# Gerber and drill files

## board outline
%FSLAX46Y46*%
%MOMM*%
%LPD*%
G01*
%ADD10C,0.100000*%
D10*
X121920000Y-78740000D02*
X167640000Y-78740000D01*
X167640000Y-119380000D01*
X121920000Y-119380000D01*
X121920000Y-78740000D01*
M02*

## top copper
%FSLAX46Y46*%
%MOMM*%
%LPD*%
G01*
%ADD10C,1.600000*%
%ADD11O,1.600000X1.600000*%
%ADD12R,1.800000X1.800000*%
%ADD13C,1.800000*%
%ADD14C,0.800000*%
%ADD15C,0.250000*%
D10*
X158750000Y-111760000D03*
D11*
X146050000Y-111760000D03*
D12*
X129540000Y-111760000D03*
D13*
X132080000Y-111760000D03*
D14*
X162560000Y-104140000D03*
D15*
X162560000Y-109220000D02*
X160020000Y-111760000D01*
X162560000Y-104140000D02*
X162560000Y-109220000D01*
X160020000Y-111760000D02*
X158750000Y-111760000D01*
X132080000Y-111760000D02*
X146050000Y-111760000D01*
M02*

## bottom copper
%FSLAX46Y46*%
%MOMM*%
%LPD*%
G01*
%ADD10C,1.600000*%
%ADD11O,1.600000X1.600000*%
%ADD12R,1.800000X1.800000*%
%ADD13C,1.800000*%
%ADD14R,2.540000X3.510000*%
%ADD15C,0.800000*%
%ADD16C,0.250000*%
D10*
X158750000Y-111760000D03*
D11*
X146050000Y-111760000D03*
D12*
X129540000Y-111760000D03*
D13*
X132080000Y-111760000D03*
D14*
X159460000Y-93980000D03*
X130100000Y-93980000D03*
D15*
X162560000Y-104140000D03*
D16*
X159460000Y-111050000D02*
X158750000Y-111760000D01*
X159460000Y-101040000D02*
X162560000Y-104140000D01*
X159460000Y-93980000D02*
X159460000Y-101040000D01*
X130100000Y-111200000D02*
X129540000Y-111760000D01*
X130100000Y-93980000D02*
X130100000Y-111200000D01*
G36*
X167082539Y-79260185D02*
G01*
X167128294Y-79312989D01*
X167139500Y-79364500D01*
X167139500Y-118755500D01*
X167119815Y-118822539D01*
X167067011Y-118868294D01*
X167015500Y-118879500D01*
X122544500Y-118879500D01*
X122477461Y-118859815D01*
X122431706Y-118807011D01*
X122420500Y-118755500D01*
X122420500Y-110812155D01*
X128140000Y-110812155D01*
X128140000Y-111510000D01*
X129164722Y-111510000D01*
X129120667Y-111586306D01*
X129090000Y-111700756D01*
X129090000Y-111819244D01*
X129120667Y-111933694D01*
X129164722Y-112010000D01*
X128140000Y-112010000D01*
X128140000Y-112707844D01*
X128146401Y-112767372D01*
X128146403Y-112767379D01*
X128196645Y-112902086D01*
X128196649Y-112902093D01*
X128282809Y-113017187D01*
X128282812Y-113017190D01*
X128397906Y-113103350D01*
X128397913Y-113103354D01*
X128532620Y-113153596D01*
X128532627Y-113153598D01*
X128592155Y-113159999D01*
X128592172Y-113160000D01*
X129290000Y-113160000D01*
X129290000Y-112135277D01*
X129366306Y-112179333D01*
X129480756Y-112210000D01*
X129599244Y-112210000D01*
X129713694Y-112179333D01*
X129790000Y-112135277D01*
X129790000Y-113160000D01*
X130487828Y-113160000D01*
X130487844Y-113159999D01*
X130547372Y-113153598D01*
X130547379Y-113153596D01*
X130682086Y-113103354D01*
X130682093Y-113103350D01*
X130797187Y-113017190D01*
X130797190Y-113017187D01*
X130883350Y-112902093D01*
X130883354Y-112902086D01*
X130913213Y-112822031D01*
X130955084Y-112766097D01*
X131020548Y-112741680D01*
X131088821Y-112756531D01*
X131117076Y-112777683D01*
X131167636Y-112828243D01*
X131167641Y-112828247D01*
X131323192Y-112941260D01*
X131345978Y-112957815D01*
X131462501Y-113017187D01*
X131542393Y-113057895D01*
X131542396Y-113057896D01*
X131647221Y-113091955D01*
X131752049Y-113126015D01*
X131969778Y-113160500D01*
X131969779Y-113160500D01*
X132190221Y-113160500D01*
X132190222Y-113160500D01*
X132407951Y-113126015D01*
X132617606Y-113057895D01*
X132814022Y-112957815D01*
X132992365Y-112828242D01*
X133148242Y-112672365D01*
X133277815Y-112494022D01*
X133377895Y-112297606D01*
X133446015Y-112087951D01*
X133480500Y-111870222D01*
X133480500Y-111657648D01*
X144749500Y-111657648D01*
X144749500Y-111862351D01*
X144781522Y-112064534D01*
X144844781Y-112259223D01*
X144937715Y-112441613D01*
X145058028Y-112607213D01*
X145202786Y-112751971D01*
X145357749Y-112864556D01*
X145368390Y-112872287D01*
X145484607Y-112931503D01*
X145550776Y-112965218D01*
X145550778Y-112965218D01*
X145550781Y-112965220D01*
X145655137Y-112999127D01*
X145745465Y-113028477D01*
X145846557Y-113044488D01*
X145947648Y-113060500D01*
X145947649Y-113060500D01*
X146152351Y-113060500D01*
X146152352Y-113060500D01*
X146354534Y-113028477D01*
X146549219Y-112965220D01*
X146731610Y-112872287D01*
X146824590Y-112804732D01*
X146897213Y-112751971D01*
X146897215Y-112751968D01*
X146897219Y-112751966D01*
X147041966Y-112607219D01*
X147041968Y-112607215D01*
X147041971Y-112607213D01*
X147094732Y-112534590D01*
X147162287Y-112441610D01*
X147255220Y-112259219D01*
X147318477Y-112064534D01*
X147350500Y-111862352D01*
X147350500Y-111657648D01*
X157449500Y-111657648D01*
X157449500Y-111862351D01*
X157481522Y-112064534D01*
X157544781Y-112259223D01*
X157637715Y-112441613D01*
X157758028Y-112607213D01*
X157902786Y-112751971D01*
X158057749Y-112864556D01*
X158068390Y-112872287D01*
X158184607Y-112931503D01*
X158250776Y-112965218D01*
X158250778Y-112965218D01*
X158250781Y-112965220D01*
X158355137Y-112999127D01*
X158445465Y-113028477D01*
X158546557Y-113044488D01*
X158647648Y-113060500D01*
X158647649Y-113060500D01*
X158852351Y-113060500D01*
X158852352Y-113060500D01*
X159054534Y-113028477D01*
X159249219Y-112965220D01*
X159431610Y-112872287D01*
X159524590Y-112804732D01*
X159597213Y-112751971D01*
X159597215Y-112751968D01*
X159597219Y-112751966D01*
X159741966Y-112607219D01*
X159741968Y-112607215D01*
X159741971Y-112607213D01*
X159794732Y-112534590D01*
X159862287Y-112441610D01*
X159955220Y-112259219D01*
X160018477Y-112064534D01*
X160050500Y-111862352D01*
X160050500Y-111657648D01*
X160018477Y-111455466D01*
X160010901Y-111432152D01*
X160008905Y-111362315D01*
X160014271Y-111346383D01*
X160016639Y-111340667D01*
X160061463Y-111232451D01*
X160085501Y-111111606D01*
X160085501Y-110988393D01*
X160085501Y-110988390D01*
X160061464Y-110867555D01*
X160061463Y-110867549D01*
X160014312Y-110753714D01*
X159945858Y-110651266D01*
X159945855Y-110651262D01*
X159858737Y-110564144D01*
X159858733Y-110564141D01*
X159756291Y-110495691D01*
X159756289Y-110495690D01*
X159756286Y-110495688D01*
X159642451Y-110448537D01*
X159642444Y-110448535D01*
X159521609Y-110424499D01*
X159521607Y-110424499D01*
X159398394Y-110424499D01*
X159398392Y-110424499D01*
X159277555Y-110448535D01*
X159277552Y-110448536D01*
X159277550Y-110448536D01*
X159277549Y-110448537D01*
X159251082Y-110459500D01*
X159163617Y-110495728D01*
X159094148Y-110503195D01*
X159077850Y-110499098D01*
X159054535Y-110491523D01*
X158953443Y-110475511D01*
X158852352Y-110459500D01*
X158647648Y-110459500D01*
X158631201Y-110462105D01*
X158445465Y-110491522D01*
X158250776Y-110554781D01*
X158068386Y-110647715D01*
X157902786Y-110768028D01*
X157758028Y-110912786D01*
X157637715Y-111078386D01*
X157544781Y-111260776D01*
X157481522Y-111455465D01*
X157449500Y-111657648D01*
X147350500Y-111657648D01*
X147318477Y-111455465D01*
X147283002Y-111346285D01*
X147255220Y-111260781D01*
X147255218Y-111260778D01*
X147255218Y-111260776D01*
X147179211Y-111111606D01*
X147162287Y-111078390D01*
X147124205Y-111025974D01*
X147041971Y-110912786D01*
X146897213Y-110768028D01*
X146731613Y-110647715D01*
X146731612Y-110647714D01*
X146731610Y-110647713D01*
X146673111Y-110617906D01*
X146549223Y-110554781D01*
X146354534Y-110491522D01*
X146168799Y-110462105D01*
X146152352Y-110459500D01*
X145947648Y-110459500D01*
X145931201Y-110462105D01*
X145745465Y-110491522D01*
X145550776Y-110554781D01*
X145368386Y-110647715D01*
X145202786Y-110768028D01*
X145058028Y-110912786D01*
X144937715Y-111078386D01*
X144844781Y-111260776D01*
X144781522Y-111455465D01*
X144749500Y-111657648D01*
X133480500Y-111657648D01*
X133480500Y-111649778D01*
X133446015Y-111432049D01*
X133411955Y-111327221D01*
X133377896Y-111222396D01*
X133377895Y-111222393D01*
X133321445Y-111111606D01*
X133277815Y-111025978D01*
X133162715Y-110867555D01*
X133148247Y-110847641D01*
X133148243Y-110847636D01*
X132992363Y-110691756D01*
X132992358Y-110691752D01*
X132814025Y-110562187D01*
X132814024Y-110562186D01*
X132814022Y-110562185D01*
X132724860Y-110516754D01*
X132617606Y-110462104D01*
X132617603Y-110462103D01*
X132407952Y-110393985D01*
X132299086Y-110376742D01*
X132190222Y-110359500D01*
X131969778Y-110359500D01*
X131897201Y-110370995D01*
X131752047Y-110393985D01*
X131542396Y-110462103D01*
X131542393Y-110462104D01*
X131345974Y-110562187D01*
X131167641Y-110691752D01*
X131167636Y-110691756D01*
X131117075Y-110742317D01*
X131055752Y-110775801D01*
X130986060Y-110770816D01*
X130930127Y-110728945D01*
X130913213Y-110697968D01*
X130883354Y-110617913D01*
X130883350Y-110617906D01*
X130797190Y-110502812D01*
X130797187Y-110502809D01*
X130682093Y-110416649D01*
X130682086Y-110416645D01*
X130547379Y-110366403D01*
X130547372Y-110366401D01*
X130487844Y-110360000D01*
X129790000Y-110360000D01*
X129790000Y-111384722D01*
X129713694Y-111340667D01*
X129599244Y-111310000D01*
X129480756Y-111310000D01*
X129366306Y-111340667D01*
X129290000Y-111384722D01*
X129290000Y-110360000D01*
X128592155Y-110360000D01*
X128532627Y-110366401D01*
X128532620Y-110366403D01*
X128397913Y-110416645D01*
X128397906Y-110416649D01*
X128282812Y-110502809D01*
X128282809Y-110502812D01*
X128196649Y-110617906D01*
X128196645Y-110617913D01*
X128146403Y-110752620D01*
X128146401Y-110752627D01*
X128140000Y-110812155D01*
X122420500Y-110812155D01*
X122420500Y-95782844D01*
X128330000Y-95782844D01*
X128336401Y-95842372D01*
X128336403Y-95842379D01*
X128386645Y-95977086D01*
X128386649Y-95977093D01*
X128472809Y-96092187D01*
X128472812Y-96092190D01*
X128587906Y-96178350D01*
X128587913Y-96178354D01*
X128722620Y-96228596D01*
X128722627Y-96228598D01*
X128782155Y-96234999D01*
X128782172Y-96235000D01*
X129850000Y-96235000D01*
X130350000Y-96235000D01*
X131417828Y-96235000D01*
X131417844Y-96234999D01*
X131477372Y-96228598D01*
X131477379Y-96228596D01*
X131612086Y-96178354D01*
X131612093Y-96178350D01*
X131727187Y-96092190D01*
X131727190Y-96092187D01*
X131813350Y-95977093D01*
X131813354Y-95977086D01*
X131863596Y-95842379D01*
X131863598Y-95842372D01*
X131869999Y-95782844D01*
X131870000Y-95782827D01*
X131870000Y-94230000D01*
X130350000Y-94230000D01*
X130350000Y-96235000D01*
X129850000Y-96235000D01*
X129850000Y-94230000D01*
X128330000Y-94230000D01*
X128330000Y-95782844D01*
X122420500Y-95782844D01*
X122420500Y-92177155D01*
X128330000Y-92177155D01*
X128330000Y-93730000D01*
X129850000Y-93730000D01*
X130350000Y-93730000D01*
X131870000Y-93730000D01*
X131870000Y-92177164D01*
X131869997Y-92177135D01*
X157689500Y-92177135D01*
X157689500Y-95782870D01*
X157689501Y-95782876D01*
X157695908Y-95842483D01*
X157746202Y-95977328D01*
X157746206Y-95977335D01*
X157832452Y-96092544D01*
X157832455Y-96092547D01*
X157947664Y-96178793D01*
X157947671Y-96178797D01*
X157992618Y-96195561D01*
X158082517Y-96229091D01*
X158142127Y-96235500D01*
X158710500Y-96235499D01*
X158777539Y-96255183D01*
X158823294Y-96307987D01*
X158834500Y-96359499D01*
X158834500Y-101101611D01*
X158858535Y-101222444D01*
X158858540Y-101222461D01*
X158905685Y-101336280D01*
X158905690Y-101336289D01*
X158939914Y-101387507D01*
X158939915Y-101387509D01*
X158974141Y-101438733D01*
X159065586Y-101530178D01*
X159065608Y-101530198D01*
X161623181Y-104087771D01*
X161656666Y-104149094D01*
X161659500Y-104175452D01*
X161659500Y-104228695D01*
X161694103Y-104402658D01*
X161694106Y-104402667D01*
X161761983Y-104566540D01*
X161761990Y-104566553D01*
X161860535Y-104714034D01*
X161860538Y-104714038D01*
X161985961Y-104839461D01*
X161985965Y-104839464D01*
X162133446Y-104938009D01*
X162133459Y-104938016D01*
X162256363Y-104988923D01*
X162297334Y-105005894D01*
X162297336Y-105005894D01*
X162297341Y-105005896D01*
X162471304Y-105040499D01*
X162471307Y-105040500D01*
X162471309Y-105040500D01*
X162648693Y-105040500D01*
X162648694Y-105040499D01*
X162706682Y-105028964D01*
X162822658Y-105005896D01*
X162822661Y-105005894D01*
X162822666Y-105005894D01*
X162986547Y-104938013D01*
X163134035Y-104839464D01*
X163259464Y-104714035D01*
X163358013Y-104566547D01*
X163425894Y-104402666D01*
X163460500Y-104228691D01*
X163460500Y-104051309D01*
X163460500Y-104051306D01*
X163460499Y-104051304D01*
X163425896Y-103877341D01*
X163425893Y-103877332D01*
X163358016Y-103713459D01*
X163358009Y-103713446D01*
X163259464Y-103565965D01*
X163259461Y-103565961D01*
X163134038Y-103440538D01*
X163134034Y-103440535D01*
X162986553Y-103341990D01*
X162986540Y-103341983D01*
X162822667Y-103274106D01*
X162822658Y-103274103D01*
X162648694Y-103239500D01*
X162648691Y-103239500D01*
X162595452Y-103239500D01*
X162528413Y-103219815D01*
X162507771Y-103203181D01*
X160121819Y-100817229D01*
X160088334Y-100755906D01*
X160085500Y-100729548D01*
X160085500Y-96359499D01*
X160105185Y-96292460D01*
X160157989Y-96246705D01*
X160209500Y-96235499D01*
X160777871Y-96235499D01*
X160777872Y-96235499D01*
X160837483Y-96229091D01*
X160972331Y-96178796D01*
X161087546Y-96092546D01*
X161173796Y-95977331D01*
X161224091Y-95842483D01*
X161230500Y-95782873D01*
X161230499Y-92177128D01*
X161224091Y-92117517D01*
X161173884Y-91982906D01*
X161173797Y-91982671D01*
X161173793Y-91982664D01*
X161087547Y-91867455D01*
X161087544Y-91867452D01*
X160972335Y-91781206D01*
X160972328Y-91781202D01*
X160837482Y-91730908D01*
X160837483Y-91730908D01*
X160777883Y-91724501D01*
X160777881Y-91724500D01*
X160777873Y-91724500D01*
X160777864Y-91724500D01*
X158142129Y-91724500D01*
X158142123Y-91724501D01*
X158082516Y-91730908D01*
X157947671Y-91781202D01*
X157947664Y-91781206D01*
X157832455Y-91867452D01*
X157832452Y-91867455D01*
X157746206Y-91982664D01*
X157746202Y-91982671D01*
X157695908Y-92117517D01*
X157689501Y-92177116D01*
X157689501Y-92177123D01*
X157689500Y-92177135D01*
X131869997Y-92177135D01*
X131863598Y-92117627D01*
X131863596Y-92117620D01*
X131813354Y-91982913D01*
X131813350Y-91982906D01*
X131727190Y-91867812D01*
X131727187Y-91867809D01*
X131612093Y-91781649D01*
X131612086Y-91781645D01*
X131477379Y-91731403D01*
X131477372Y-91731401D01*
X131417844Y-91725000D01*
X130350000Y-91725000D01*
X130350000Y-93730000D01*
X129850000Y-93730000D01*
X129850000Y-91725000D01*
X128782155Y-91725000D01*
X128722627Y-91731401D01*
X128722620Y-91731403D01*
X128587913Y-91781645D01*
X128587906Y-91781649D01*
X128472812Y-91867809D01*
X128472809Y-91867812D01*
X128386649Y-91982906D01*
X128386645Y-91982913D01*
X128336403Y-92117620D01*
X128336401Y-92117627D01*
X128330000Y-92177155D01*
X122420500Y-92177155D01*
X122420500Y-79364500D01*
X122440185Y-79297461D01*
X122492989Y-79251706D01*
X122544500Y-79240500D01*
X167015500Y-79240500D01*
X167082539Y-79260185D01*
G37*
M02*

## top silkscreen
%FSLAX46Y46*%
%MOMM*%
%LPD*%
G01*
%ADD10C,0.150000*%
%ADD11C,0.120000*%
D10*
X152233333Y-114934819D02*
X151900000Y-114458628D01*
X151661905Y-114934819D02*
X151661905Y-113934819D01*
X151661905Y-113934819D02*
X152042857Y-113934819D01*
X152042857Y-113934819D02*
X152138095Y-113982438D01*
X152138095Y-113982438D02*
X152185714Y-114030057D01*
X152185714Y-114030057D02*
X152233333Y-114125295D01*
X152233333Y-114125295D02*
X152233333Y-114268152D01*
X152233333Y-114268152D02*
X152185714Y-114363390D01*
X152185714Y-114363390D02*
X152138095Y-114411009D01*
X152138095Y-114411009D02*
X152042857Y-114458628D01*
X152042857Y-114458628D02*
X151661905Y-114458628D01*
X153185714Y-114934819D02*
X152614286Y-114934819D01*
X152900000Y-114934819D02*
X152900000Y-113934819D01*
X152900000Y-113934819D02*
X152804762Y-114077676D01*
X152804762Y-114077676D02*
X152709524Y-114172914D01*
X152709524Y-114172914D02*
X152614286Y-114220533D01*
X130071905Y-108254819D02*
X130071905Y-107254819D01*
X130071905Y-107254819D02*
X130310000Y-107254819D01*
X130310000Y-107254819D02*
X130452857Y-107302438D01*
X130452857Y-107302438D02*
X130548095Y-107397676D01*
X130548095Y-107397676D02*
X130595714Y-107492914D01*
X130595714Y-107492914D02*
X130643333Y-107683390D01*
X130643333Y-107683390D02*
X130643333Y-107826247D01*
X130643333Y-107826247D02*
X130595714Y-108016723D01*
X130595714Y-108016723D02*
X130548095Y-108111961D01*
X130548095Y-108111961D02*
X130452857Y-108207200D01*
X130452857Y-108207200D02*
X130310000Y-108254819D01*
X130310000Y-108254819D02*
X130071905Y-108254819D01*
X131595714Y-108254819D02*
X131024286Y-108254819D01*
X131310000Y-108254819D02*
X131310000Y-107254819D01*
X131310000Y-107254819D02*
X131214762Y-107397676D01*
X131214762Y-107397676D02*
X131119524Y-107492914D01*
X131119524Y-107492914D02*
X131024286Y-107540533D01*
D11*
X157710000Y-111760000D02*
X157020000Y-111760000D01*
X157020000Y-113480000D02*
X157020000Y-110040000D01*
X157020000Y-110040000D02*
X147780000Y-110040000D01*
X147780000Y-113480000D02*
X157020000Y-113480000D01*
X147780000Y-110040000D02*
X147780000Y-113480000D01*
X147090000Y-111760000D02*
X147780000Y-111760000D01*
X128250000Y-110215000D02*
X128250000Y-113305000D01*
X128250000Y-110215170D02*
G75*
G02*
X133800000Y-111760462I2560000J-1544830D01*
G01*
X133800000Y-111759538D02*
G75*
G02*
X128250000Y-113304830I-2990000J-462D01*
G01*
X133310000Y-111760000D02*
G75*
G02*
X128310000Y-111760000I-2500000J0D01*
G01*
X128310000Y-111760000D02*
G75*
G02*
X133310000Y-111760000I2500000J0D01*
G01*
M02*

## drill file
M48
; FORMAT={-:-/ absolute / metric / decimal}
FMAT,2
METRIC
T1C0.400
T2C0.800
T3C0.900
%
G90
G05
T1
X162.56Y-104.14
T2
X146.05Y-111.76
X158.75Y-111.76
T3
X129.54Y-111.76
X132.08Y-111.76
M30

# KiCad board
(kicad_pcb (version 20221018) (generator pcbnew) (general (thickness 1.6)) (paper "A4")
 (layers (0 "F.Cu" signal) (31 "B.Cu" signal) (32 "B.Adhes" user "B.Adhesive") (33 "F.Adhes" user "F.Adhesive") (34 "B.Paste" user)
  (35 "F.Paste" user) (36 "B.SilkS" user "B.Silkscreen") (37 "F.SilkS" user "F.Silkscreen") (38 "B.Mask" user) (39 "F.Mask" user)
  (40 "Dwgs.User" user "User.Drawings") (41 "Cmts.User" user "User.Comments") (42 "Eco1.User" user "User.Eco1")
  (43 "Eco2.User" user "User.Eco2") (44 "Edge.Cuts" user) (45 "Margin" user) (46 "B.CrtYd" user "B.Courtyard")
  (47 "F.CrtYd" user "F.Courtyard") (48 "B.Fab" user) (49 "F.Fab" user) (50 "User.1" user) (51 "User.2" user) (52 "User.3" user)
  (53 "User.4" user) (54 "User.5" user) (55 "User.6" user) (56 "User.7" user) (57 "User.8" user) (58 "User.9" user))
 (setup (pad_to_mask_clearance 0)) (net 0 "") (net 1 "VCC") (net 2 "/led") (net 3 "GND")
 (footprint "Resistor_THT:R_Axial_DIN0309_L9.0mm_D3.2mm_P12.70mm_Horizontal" (layer "F.Cu") (at 158.75 111.76 180)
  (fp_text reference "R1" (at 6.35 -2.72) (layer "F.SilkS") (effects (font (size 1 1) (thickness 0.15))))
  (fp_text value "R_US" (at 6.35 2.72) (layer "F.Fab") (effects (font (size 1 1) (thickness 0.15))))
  (fp_line (start 1.04 0) (end 1.73 0) (stroke (width 0.12) (type solid)) (layer "F.SilkS"))
  (fp_line (start 1.73 -1.72) (end 1.73 1.72) (stroke (width 0.12) (type solid)) (layer "F.SilkS"))
  (fp_line (start 1.73 1.72) (end 10.97 1.72) (stroke (width 0.12) (type solid)) (layer "F.SilkS"))
  (fp_line (start 10.97 -1.72) (end 1.73 -1.72) (stroke (width 0.12) (type solid)) (layer "F.SilkS"))
  (fp_line (start 10.97 1.72) (end 10.97 -1.72) (stroke (width 0.12) (type solid)) (layer "F.SilkS"))
  (fp_line (start 11.66 0) (end 10.97 0) (stroke (width 0.12) (type solid)) (layer "F.SilkS"))
  (pad "1" thru_hole circle (at 0 0 180) (size 1.6 1.6) (drill 0.8) (layers "*.Cu" "*.Mask") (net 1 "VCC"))
  (pad "2" thru_hole oval (at 12.7 0 180) (size 1.6 1.6) (drill 0.8) (layers "*.Cu" "*.Mask") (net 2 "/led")))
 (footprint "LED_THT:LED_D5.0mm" (layer "F.Cu") (at 129.54 111.76)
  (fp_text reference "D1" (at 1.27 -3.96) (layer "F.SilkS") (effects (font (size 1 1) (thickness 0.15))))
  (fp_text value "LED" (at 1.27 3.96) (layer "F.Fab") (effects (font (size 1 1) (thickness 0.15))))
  (fp_line (start -1.29 -1.545) (end -1.29 1.545) (stroke (width 0.12) (type solid)) (layer "F.SilkS"))
  (fp_arc (start -1.29 -1.54483) (mid 2.072002 -2.880433) (end 4.26 0.000462) (stroke (width 0.12) (type solid)) (layer "F.SilkS"))
  (fp_arc (start 4.26 -0.000462) (mid 2.072002 2.880433) (end -1.29 1.54483) (stroke (width 0.12) (type solid)) (layer "F.SilkS"))
  (fp_circle (center 1.27 0) (end 3.77 0) (stroke (width 0.12) (type solid)) (fill none) (layer "F.SilkS"))
  (pad "1" thru_hole rect (at 0 0) (size 1.8 1.8) (drill 0.9) (layers "*.Cu" "*.Mask") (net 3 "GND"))
  (pad "2" thru_hole circle (at 2.54 0) (size 1.8 1.8) (drill 0.9) (layers "*.Cu" "*.Mask") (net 2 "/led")))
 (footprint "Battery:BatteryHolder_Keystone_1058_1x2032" (layer "B.Cu") (at 144.78 93.98 180)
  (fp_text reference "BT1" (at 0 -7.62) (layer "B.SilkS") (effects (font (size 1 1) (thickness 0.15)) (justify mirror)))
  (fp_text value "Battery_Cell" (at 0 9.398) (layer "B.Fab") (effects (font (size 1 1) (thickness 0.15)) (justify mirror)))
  (pad "1" smd rect (at -14.68 0 180) (size 2.54 3.51) (layers "B.Cu" "B.Paste" "B.Mask") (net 1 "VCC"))
  (pad "2" smd rect (at 14.68 0 180) (size 2.54 3.51) (layers "B.Cu" "B.Paste" "B.Mask") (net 3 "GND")))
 (gr_rect (start 121.92 78.74) (end 167.64 119.38) (stroke (width 0.1) (type default)) (fill none) (layer "Edge.Cuts"))
 (segment (start 162.56 109.22) (end 160.02 111.76) (width 0.25) (layer "F.Cu") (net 1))
 (segment (start 162.56 104.14) (end 162.56 109.22) (width 0.25) (layer "F.Cu") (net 1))
 (segment (start 160.02 111.76) (end 158.75 111.76) (width 0.25) (layer "F.Cu") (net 1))
 (via (at 162.56 104.14) (size 0.8) (drill 0.4) (layers "F.Cu" "B.Cu") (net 1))
 (segment (start 159.46 111.05) (end 158.75 111.76) (width 0.25) (layer "B.Cu") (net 1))
 (segment (start 159.46 101.04) (end 162.56 104.14) (width 0.25) (layer "B.Cu") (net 1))
 (segment (start 159.46 93.98) (end 159.46 101.04) (width 0.25) (layer "B.Cu") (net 1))
 (segment (start 130.1 111.2) (end 129.54 111.76) (width 0.25) (layer "B.Cu") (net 3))
 (segment (start 130.1 93.98) (end 130.1 111.2) (width 0.25) (layer "B.Cu") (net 3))
 (segment (start 132.08 111.76) (end 146.05 111.76) (width 0.25) (layer "F.Cu") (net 2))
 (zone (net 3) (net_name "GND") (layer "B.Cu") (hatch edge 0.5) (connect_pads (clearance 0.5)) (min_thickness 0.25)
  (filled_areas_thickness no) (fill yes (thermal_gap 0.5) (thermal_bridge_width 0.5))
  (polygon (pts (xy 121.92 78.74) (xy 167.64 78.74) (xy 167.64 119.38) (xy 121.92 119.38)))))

